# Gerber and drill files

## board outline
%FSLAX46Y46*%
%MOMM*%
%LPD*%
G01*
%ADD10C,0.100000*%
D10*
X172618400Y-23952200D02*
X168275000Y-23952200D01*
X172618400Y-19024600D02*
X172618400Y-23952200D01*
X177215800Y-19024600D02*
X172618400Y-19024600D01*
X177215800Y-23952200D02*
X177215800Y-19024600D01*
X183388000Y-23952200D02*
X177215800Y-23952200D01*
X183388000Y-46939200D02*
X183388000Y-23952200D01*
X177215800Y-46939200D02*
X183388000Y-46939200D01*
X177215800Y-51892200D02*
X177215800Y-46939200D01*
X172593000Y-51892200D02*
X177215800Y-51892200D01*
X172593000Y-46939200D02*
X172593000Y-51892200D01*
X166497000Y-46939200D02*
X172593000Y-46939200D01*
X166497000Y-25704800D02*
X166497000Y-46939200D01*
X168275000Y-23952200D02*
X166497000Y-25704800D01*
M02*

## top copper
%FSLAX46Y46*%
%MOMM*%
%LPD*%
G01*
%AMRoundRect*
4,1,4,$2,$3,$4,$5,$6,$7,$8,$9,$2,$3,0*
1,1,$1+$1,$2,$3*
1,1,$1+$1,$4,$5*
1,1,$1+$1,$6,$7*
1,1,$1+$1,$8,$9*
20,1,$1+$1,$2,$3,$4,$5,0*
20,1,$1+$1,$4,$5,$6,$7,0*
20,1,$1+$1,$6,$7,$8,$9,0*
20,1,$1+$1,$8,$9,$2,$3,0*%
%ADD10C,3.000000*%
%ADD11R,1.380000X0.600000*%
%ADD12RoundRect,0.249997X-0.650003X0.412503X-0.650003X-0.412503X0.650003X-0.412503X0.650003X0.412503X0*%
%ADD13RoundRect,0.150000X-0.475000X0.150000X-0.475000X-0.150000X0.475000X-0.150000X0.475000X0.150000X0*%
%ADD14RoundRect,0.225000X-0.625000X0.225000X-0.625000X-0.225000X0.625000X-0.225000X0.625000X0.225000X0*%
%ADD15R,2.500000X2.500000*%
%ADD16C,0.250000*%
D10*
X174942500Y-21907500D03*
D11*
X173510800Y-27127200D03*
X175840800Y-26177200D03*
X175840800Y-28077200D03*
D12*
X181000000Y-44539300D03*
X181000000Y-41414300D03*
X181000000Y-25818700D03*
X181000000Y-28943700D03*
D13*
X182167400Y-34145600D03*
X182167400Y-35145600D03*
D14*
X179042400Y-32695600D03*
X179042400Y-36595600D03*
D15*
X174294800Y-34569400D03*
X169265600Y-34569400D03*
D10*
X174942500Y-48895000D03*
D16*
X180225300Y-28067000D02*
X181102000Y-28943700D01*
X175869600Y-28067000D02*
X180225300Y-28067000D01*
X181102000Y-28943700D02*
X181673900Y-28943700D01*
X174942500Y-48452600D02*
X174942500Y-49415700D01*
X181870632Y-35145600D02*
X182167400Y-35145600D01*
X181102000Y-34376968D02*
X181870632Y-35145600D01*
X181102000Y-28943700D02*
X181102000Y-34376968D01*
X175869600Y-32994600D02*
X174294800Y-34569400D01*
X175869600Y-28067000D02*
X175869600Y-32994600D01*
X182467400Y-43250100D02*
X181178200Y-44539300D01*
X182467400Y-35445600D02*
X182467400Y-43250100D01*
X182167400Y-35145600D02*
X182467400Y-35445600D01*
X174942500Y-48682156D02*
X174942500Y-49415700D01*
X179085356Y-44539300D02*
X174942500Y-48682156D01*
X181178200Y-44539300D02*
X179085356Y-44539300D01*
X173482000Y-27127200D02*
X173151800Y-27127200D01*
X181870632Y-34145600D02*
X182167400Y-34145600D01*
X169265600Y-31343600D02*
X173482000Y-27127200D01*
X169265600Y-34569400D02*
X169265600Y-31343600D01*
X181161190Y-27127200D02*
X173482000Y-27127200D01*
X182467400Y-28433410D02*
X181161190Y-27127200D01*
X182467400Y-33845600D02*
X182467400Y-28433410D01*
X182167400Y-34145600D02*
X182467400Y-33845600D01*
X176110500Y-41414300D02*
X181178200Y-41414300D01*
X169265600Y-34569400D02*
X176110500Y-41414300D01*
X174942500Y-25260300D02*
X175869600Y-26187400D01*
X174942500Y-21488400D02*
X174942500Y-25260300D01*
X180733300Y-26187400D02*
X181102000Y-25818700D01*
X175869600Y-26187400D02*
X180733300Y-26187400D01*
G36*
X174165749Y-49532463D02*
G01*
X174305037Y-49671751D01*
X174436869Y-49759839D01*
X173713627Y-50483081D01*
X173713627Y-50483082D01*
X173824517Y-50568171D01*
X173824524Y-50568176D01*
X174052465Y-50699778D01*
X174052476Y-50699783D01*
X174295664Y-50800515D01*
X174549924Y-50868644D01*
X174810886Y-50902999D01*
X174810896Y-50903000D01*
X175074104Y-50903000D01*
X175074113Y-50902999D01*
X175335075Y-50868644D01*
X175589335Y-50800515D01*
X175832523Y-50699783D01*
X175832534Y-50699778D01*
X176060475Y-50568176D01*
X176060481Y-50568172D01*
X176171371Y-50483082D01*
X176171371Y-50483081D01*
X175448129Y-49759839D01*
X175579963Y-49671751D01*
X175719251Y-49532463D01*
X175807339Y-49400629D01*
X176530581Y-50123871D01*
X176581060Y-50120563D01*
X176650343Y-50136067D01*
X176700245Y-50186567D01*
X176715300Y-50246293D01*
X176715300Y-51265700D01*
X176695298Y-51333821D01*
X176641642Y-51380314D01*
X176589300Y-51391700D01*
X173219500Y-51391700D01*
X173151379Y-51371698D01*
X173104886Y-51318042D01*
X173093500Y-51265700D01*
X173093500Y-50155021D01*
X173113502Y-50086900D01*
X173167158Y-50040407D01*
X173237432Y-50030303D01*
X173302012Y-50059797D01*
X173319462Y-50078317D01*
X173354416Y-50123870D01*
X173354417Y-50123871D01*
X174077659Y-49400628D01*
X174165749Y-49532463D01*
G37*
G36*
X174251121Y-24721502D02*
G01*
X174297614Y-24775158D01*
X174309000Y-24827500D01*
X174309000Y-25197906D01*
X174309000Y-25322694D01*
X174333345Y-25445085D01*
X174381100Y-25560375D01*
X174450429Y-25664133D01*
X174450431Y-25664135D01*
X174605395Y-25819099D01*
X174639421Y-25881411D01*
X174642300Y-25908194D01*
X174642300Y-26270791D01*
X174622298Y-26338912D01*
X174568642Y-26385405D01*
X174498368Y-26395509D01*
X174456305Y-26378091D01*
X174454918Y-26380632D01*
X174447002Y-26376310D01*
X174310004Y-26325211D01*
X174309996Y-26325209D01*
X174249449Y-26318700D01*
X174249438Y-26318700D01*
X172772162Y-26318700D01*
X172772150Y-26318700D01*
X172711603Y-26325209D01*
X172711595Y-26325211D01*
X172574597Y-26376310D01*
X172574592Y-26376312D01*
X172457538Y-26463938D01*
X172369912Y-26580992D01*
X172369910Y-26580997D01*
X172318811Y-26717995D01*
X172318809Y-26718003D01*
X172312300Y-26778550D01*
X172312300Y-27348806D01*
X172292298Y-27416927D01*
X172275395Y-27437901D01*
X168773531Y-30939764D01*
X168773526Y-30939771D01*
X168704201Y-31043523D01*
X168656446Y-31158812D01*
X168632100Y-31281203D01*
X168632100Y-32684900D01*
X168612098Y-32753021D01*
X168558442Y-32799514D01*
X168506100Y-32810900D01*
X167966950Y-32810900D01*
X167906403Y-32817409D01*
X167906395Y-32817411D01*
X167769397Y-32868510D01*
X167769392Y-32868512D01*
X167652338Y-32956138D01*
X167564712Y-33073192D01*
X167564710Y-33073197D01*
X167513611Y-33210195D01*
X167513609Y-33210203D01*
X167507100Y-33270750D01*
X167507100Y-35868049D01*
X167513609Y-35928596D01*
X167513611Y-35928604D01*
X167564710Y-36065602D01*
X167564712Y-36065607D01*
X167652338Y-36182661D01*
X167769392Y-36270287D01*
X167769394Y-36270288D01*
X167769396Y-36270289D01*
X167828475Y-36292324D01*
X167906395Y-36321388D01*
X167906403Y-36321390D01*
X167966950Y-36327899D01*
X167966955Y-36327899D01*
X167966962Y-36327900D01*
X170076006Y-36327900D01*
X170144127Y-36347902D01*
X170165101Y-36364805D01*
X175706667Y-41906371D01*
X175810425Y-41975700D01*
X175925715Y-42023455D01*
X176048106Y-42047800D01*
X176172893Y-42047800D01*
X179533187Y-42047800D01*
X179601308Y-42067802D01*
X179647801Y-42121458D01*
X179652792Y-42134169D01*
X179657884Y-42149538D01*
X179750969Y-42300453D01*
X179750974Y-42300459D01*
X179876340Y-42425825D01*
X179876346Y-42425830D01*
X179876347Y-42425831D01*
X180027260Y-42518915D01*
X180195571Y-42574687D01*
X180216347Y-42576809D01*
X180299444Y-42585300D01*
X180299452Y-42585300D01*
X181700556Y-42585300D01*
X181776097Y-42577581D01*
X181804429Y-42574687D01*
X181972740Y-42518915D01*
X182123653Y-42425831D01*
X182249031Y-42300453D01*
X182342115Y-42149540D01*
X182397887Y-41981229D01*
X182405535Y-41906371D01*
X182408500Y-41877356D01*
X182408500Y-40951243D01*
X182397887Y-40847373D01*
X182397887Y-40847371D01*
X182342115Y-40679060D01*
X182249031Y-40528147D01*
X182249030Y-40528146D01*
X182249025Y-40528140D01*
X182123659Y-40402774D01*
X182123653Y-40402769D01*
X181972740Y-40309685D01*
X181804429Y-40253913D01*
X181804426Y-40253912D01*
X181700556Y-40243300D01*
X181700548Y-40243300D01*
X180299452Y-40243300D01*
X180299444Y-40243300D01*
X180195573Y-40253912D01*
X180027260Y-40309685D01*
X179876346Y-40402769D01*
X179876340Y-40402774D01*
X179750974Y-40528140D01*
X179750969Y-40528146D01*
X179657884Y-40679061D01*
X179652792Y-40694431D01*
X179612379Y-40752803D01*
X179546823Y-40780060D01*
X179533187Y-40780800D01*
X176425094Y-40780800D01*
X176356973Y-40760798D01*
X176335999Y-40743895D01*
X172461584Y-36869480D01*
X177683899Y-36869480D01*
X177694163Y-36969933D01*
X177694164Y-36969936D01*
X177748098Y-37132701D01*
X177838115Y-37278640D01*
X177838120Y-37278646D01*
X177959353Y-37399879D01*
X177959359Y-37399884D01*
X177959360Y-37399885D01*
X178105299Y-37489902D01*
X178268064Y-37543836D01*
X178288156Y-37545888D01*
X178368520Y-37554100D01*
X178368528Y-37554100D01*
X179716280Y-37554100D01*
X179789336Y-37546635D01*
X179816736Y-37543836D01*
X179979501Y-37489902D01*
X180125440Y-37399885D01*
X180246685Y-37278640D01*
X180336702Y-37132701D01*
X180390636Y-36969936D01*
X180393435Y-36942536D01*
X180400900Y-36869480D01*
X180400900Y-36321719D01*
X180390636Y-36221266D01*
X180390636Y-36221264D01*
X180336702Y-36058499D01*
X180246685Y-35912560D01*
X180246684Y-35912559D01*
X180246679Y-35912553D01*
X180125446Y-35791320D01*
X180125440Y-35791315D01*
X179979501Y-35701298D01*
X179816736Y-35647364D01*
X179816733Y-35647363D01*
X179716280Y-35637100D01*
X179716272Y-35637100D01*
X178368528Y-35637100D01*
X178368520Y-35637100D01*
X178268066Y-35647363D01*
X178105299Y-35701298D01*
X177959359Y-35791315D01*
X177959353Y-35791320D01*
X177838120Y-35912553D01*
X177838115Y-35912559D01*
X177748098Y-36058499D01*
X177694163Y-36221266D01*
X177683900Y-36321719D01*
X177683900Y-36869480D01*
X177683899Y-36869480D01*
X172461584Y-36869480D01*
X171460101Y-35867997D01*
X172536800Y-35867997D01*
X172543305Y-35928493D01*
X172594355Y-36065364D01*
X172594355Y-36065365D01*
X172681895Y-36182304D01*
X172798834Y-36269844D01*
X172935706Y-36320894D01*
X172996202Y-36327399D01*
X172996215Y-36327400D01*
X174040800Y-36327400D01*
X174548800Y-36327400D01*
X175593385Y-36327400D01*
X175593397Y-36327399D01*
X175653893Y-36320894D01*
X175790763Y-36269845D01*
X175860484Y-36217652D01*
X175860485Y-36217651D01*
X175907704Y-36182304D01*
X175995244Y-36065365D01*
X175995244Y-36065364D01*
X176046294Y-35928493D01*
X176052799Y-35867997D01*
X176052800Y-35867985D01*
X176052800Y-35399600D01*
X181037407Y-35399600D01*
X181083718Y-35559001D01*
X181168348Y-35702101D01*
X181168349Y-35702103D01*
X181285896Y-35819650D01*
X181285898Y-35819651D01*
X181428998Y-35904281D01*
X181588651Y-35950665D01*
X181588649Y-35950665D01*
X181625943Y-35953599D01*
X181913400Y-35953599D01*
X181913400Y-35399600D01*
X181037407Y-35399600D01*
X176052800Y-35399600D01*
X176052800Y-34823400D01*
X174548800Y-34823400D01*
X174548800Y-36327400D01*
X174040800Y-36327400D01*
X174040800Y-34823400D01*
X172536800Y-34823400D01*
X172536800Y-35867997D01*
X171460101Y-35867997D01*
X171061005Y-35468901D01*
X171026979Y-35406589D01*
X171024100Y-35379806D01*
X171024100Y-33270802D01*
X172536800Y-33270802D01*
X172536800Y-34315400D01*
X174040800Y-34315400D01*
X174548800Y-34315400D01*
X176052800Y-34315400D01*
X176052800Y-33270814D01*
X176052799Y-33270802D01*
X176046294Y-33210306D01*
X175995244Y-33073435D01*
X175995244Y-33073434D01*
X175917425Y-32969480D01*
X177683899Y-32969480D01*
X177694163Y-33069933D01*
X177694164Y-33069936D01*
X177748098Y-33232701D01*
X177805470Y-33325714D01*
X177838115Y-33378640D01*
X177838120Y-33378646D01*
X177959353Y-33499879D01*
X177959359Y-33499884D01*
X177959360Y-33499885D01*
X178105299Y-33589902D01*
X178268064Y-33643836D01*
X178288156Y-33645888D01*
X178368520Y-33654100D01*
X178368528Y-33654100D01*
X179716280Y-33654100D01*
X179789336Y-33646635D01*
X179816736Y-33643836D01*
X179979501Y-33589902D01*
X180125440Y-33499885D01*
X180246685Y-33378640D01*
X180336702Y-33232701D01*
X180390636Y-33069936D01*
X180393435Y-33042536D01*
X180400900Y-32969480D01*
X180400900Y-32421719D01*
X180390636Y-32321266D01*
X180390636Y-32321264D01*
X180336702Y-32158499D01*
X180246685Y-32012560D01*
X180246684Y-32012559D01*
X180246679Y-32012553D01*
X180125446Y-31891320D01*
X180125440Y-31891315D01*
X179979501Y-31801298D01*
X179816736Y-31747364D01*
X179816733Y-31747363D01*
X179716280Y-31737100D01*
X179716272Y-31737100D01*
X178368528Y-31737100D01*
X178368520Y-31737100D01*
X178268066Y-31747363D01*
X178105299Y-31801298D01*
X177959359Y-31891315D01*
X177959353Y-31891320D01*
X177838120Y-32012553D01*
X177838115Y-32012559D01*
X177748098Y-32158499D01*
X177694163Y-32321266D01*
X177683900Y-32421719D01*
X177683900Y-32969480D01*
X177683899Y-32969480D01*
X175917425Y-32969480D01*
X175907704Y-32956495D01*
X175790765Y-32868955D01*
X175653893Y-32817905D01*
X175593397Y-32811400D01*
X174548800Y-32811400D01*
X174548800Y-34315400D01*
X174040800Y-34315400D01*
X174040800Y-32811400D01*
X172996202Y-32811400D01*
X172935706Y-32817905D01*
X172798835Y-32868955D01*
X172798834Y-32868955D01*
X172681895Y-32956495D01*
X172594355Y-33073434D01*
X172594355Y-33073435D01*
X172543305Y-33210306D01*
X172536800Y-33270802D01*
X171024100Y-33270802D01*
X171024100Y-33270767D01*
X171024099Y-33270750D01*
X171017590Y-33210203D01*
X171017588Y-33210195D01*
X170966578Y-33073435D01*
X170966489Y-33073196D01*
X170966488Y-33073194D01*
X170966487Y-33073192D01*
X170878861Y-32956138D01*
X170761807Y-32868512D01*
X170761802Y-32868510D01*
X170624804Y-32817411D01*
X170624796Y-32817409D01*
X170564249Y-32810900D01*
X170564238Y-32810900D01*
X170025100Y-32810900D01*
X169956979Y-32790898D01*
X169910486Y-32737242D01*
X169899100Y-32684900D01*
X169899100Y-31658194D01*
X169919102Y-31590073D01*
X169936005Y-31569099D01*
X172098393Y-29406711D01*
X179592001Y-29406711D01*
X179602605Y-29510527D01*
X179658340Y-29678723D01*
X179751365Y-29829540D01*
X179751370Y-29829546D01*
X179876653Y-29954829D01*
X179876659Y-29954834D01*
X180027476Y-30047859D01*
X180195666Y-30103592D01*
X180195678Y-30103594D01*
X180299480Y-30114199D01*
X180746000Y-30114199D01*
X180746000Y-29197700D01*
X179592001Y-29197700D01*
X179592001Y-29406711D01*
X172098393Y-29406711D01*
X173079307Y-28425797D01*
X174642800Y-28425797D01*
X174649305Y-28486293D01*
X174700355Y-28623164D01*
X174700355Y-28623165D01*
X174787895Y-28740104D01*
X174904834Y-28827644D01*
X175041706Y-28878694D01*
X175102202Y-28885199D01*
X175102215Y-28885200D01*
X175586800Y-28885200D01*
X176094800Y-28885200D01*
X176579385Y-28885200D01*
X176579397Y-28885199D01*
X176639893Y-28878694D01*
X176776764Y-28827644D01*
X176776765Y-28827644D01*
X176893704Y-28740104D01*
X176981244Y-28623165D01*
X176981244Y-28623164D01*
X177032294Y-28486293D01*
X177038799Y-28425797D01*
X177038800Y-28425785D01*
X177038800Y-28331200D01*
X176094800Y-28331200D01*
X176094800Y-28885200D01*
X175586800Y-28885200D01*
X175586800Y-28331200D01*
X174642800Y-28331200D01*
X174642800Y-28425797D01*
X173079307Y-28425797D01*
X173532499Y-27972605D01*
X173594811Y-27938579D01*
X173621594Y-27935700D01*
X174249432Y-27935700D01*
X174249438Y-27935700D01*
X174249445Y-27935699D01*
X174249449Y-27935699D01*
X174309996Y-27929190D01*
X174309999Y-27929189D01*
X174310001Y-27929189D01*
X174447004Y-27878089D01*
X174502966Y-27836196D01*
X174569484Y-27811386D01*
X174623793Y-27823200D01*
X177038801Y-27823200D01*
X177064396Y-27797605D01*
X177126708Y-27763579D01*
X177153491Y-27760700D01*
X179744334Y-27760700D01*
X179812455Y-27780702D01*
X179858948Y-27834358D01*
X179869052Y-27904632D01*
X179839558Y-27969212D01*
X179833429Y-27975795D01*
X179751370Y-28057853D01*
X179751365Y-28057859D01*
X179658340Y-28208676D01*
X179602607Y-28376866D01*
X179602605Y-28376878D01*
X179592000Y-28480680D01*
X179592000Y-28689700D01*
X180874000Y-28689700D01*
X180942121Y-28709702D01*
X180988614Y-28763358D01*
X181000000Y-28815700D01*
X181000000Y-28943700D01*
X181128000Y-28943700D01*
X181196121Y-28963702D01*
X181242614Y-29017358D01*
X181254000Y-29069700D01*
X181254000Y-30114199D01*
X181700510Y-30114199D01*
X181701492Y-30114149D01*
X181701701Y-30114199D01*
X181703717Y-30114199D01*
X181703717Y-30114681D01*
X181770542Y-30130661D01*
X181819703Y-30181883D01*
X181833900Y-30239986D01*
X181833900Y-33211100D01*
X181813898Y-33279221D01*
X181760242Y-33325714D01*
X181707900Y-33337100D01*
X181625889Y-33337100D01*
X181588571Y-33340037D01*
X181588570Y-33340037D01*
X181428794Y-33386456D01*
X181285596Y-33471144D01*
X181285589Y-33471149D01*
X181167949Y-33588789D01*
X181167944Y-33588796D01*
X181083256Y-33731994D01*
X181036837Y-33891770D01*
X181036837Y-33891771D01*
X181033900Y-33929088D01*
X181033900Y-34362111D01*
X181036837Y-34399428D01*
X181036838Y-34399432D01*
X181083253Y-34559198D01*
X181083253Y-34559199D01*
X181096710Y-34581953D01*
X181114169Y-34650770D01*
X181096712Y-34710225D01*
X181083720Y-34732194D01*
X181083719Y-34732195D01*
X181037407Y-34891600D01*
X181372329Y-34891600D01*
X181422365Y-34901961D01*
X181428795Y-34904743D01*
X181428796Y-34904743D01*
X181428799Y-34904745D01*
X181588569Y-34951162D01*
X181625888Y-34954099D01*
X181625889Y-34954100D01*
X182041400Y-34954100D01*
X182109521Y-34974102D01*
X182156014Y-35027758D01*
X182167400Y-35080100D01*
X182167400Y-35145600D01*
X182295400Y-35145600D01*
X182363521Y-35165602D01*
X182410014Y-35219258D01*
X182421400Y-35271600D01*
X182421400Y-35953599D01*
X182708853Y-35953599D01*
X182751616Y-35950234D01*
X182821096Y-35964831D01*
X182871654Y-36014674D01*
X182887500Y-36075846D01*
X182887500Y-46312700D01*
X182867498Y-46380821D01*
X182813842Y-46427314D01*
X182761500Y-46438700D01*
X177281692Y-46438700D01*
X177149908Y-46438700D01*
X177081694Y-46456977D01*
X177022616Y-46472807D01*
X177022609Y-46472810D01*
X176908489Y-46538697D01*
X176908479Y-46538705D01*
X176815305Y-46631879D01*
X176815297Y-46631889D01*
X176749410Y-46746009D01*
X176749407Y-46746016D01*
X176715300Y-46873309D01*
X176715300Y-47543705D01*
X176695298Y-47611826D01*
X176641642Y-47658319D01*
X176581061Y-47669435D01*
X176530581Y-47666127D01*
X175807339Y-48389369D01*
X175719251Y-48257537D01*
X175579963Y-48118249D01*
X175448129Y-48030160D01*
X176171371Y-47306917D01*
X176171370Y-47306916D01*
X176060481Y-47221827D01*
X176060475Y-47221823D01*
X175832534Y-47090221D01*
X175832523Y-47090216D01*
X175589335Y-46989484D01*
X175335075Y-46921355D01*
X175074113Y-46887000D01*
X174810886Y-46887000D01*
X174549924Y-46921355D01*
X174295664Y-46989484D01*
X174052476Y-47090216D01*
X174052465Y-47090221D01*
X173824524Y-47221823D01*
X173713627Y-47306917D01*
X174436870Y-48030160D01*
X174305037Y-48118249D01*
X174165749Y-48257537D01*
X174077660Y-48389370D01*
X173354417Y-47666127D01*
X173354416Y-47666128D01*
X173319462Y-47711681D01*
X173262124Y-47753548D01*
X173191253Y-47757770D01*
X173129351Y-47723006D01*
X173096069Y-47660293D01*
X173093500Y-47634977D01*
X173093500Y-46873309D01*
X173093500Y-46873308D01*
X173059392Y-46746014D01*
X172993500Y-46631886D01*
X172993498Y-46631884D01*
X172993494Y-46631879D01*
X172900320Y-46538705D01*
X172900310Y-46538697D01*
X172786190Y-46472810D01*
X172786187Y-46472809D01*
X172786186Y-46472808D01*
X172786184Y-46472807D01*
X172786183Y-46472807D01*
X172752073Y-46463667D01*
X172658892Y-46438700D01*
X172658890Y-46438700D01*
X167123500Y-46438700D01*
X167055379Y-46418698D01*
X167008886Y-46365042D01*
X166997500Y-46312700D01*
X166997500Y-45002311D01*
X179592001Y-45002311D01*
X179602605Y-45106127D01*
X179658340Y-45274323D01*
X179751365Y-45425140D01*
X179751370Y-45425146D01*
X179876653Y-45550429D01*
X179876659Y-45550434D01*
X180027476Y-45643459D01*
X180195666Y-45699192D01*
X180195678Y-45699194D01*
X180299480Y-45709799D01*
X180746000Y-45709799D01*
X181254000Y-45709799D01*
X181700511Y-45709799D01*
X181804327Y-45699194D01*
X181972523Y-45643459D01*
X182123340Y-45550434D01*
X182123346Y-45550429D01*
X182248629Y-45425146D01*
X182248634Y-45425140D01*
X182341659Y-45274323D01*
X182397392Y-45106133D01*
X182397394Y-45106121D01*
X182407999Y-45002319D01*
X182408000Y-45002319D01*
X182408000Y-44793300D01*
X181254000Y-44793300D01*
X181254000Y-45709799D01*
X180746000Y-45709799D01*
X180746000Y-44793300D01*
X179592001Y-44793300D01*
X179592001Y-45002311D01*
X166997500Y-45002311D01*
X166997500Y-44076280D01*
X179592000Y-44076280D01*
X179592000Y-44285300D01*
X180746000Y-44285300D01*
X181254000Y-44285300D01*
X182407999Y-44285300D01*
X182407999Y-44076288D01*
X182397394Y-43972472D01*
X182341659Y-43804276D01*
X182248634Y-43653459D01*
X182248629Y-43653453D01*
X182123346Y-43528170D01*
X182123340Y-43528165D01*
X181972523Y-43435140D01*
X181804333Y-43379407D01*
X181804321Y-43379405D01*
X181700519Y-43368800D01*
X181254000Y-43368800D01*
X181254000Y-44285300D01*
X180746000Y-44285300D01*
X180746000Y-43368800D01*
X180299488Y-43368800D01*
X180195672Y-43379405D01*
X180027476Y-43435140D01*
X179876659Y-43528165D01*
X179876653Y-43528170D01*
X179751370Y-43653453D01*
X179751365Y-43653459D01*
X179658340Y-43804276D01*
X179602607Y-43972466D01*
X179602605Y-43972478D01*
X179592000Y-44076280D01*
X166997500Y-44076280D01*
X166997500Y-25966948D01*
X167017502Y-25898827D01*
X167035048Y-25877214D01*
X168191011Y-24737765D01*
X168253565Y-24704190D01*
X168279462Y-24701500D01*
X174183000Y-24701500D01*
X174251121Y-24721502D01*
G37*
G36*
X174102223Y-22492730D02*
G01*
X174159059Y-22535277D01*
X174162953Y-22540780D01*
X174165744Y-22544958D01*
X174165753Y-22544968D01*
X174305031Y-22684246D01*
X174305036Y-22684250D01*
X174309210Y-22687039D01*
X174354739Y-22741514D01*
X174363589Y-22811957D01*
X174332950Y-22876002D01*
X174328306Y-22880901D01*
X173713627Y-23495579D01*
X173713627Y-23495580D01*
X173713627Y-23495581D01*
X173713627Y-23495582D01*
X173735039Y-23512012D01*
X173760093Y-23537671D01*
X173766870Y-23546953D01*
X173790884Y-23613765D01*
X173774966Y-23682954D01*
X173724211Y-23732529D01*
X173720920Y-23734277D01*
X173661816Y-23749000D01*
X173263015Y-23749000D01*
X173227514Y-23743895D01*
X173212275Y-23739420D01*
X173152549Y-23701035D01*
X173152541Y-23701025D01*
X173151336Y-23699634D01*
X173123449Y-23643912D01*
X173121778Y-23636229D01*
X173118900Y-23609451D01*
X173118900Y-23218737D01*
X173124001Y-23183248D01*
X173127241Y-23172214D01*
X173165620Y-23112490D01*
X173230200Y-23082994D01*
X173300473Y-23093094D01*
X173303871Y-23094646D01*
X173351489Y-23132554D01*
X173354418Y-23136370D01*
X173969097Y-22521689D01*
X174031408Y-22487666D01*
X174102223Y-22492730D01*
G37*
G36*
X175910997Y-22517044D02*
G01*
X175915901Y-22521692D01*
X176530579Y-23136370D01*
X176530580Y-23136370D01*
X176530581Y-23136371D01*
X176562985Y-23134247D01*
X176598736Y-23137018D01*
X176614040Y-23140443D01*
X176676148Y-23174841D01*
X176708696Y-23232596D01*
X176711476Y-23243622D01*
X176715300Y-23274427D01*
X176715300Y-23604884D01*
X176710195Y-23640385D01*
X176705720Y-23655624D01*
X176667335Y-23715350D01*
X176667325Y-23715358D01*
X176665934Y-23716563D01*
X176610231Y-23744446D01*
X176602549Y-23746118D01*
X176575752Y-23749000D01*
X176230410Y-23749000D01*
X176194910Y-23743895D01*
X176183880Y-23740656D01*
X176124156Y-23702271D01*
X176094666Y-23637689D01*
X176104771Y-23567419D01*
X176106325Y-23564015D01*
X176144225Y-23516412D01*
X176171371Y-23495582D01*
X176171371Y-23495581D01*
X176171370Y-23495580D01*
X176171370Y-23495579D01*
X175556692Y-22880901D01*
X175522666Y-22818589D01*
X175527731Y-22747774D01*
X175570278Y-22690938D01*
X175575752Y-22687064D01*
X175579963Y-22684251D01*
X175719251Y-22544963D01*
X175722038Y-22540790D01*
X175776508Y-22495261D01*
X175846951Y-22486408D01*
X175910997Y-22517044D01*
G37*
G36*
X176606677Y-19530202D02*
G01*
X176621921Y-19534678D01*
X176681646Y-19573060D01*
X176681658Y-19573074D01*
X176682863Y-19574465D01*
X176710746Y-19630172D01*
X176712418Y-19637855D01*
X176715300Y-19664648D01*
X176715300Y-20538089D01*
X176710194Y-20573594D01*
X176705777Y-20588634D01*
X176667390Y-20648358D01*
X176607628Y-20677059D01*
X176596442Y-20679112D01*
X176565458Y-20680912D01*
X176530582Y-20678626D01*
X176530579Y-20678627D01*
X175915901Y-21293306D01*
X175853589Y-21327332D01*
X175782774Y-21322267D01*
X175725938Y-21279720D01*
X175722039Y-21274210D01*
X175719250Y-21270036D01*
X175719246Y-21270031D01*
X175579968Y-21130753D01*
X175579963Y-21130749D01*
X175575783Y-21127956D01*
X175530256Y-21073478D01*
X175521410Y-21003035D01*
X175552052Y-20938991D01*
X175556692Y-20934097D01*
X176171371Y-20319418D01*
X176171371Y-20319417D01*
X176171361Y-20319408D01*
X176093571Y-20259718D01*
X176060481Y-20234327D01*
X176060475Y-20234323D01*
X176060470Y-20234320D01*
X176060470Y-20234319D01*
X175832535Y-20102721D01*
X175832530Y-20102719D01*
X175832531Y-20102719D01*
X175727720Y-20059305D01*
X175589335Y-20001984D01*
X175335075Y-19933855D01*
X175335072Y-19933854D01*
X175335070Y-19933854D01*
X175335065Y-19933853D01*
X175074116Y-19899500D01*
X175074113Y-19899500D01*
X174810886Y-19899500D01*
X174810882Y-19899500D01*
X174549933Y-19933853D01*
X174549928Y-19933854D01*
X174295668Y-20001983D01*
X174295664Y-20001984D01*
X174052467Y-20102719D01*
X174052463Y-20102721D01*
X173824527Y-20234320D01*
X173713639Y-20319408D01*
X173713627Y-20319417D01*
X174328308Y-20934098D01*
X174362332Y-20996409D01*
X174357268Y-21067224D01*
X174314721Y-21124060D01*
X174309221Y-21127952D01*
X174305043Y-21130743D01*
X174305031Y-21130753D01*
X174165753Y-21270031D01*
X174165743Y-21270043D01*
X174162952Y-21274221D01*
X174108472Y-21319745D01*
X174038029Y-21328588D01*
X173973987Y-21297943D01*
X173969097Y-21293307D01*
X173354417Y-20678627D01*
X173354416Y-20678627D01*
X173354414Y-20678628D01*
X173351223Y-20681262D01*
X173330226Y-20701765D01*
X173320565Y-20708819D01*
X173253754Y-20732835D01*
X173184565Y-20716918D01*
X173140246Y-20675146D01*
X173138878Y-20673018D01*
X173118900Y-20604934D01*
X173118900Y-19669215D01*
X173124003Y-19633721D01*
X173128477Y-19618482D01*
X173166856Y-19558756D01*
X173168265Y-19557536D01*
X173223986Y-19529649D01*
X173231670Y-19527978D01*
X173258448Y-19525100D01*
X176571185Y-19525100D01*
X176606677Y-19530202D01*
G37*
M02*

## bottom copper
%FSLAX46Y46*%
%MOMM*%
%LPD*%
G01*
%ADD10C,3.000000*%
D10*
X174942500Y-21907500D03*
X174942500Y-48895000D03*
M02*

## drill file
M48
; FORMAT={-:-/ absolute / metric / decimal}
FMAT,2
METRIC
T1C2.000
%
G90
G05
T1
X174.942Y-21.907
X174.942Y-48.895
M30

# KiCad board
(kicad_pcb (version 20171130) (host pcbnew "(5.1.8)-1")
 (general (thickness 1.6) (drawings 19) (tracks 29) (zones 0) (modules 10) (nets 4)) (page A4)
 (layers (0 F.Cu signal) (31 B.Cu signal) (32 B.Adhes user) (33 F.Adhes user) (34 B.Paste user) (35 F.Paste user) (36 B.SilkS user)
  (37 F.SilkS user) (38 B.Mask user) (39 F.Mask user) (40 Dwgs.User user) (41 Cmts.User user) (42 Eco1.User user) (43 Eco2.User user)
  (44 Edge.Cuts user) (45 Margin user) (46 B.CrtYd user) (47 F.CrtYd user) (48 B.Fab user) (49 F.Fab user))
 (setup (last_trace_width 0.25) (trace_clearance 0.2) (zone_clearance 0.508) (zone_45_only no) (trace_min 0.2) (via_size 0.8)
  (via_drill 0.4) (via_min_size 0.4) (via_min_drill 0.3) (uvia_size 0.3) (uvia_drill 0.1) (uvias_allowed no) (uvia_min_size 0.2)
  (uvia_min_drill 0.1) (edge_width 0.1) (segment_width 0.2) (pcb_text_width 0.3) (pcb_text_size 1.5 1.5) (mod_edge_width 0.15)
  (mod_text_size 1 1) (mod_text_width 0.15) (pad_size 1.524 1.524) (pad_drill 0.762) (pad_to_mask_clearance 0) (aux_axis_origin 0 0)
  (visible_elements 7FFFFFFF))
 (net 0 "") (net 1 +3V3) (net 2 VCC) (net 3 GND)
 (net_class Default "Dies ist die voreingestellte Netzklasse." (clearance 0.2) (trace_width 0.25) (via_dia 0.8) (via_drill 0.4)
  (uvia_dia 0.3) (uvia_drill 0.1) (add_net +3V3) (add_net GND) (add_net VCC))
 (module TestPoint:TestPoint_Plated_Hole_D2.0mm (layer F.Cu) (at 174.9425 21.9075)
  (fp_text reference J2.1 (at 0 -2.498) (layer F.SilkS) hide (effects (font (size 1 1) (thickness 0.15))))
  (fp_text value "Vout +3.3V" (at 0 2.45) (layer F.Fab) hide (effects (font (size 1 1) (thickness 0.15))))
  (pad 1 thru_hole circle (at 0 0) (size 3 3) (drill 2) (layers *.Cu *.Mask) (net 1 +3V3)))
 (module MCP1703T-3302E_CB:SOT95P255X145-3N (layer F.Cu) (at 174.6758 27.1272 180)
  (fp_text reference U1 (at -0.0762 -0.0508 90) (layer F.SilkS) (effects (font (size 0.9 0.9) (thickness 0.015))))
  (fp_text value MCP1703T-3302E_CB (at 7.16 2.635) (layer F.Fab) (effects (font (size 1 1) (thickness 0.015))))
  (pad 3 smd rect (at 1.165 0 180) (size 1.38 0.6) (layers F.Cu F.Paste F.Mask) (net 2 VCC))
  (pad 2 smd rect (at -1.165 0.95 180) (size 1.38 0.6) (layers F.Cu F.Paste F.Mask) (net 1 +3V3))
  (pad 1 smd rect (at -1.165 -0.95 180) (size 1.38 0.6) (layers F.Cu F.Paste F.Mask) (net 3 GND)))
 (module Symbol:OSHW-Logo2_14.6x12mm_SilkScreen (layer B.Cu) (at 174.9425 35.4457 270)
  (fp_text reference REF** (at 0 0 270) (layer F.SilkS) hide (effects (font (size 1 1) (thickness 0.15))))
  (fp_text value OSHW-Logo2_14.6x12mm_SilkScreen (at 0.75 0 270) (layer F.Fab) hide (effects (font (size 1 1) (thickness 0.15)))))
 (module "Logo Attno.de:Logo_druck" (layer F.Cu) (at 171.7548 41.7576)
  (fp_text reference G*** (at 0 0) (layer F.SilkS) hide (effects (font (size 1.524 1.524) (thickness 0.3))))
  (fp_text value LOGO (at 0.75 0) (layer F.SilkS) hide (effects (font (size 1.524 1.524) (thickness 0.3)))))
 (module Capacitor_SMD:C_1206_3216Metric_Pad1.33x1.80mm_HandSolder (layer F.Cu) (at 181 42.9768 270)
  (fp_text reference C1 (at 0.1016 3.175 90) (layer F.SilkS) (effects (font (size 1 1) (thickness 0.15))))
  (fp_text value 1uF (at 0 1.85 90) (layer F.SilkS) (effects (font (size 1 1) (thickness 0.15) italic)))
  (pad 2 smd roundrect (at 1.5625 0 270) (size 1.325 1.8) (layers F.Cu F.Paste F.Mask) (roundrect_rratio 0.1886769811320755) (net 3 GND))
  (pad 1 smd roundrect (at -1.5625 0 270) (size 1.325 1.8) (layers F.Cu F.Paste F.Mask) (roundrect_rratio 0.1886769811320755) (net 2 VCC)))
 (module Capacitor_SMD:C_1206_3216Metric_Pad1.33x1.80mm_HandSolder (layer F.Cu) (at 181 27.3812 270)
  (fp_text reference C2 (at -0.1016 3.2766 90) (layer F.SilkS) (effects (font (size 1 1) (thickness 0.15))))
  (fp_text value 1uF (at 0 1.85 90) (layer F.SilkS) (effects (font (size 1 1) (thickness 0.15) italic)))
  (pad 1 smd roundrect (at -1.5625 0 270) (size 1.325 1.8) (layers F.Cu F.Paste F.Mask) (roundrect_rratio 0.1886769811320755) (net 1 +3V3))
  (pad 2 smd roundrect (at 1.5625 0 270) (size 1.325 1.8) (layers F.Cu F.Paste F.Mask) (roundrect_rratio 0.1886769811320755) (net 3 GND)))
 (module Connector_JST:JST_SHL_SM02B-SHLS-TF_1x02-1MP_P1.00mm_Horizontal (layer F.Cu) (at 180.4924 34.6456 270)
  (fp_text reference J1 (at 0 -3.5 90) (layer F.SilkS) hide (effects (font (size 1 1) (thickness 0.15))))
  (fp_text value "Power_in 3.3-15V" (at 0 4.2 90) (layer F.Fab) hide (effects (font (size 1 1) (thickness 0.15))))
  (pad 1 smd roundrect (at -0.5 -1.675 270) (size 0.6 1.25) (layers F.Cu F.Paste F.Mask) (roundrect_rratio 0.25) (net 2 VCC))
  (pad 2 smd roundrect (at 0.5 -1.675 270) (size 0.6 1.25) (layers F.Cu F.Paste F.Mask) (roundrect_rratio 0.25) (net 3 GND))
  (pad MP smd roundrect (at -1.95 1.45 270) (size 0.9 1.7) (layers F.Cu F.Paste F.Mask) (roundrect_rratio 0.25))
  (pad MP smd roundrect (at 1.95 1.45 270) (size 0.9 1.7) (layers F.Cu F.Paste F.Mask) (roundrect_rratio 0.25)))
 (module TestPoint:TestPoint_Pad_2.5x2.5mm (layer F.Cu) (at 174.2948 34.5694)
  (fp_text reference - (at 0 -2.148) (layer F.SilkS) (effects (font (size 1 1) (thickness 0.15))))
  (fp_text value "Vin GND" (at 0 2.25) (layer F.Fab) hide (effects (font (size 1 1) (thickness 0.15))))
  (pad 1 smd rect (at 0 0) (size 2.5 2.5) (layers F.Cu F.Mask) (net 3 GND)))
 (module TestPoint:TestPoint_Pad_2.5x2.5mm (layer F.Cu) (at 169.2656 34.5694)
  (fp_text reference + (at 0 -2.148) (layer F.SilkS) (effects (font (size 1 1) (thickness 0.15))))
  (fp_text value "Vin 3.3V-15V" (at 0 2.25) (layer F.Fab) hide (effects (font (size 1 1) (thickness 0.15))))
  (pad 1 smd rect (at 0 0) (size 2.5 2.5) (layers F.Cu F.Mask) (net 2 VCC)))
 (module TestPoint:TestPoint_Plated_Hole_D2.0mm (layer F.Cu) (at 174.9425 48.895)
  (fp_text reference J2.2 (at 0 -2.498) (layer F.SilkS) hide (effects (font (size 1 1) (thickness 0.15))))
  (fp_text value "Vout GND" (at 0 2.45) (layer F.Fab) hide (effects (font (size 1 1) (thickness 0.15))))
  (pad 1 thru_hole circle (at 0 0) (size 3 3) (drill 2) (layers *.Cu *.Mask) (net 3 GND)))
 (gr_line (start 172.6184 23.9522) (end 168.275 23.9522) (layer Edge.Cuts) (width 0.1))
 (gr_line (start 172.6184 19.0246) (end 172.6184 23.9522) (layer Edge.Cuts) (width 0.1))
 (gr_line (start 177.2158 19.0246) (end 172.6184 19.0246) (layer Edge.Cuts) (width 0.1))
 (gr_line (start 177.2158 23.9522) (end 177.2158 19.0246) (layer Edge.Cuts) (width 0.1))
 (gr_line (start 183.388 23.9522) (end 177.2158 23.9522) (layer Edge.Cuts) (width 0.1))
 (gr_line (start 183.388 46.9392) (end 183.388 23.9522) (layer Edge.Cuts) (width 0.1))
 (gr_line (start 177.2158 46.9392) (end 183.388 46.9392) (layer Edge.Cuts) (width 0.1))
 (gr_line (start 177.2158 51.8922) (end 177.2158 46.9392) (layer Edge.Cuts) (width 0.1))
 (gr_line (start 172.593 51.8922) (end 177.2158 51.8922) (layer Edge.Cuts) (width 0.1))
 (gr_line (start 172.593 46.9392) (end 172.593 51.8922) (layer Edge.Cuts) (width 0.1))
 (gr_line (start 166.497 46.9392) (end 172.593 46.9392) (layer Edge.Cuts) (width 0.1))
 (gr_line (start 166.497 25.7048) (end 166.497 46.9392) (layer Edge.Cuts) (width 0.1))
 (gr_line (start 168.275 23.9522) (end 166.497 25.7048) (layer Edge.Cuts) (width 0.1))
 (segment (start 180.2253 28.067) (end 181.102 28.9437) (width 0.25) (layer F.Cu) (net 3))
 (segment (start 175.8696 28.067) (end 180.2253 28.067) (width 0.25) (layer F.Cu) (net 3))
 (segment (start 181.102 28.9437) (end 181.6739 28.9437) (width 0.25) (layer F.Cu) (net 3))
 (segment (start 174.9425 48.4526) (end 174.9425 49.4157) (width 0.25) (layer F.Cu) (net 3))
 (segment (start 181.870632 35.1456) (end 182.1674 35.1456) (width 0.25) (layer F.Cu) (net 3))
 (segment (start 181.102 34.376968) (end 181.870632 35.1456) (width 0.25) (layer F.Cu) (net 3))
 (segment (start 181.102 28.9437) (end 181.102 34.376968) (width 0.25) (layer F.Cu) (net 3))
 (segment (start 175.8696 32.9946) (end 174.2948 34.5694) (width 0.25) (layer F.Cu) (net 3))
 (segment (start 175.8696 28.067) (end 175.8696 32.9946) (width 0.25) (layer F.Cu) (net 3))
 (segment (start 182.4674 43.2501) (end 181.1782 44.5393) (width 0.25) (layer F.Cu) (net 3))
 (segment (start 182.4674 35.4456) (end 182.4674 43.2501) (width 0.25) (layer F.Cu) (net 3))
 (segment (start 182.1674 35.1456) (end 182.4674 35.4456) (width 0.25) (layer F.Cu) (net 3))
 (segment (start 174.9425 48.682156) (end 174.9425 49.4157) (width 0.25) (layer F.Cu) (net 3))
 (segment (start 179.085356 44.5393) (end 174.9425 48.682156) (width 0.25) (layer F.Cu) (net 3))
 (segment (start 181.1782 44.5393) (end 179.085356 44.5393) (width 0.25) (layer F.Cu) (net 3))
 (segment (start 173.482 27.1272) (end 173.1518 27.1272) (width 0.25) (layer F.Cu) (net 2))
 (segment (start 181.870632 34.1456) (end 182.1674 34.1456) (width 0.25) (layer F.Cu) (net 2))
 (segment (start 169.2656 31.3436) (end 173.482 27.1272) (width 0.25) (layer F.Cu) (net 2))
 (segment (start 169.2656 34.5694) (end 169.2656 31.3436) (width 0.25) (layer F.Cu) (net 2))
 (segment (start 181.16119 27.1272) (end 173.482 27.1272) (width 0.25) (layer F.Cu) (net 2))
 (segment (start 182.4674 28.43341) (end 181.16119 27.1272) (width 0.25) (layer F.Cu) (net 2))
 (segment (start 182.4674 33.8456) (end 182.4674 28.43341) (width 0.25) (layer F.Cu) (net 2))
 (segment (start 182.1674 34.1456) (end 182.4674 33.8456) (width 0.25) (layer F.Cu) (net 2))
 (segment (start 176.1105 41.4143) (end 181.1782 41.4143) (width 0.25) (layer F.Cu) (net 2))
 (segment (start 169.2656 34.5694) (end 176.1105 41.4143) (width 0.25) (layer F.Cu) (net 2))
 (segment (start 174.9425 25.2603) (end 175.8696 26.1874) (width 0.25) (layer F.Cu) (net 1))
 (segment (start 174.9425 21.4884) (end 174.9425 25.2603) (width 0.25) (layer F.Cu) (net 1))
 (segment (start 180.7333 26.1874) (end 181.102 25.8187) (width 0.25) (layer F.Cu) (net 1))
 (segment (start 175.8696 26.1874) (end 180.7333 26.1874) (width 0.25) (layer F.Cu) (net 1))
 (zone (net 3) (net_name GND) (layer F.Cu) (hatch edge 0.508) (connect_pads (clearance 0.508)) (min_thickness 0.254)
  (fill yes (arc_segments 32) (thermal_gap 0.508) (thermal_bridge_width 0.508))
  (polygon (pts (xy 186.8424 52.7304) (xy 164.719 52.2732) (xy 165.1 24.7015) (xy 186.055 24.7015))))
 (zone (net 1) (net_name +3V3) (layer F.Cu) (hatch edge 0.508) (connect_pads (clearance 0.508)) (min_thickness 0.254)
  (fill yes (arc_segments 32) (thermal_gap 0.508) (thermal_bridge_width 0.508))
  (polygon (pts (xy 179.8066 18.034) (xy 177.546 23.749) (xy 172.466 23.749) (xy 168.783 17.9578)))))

